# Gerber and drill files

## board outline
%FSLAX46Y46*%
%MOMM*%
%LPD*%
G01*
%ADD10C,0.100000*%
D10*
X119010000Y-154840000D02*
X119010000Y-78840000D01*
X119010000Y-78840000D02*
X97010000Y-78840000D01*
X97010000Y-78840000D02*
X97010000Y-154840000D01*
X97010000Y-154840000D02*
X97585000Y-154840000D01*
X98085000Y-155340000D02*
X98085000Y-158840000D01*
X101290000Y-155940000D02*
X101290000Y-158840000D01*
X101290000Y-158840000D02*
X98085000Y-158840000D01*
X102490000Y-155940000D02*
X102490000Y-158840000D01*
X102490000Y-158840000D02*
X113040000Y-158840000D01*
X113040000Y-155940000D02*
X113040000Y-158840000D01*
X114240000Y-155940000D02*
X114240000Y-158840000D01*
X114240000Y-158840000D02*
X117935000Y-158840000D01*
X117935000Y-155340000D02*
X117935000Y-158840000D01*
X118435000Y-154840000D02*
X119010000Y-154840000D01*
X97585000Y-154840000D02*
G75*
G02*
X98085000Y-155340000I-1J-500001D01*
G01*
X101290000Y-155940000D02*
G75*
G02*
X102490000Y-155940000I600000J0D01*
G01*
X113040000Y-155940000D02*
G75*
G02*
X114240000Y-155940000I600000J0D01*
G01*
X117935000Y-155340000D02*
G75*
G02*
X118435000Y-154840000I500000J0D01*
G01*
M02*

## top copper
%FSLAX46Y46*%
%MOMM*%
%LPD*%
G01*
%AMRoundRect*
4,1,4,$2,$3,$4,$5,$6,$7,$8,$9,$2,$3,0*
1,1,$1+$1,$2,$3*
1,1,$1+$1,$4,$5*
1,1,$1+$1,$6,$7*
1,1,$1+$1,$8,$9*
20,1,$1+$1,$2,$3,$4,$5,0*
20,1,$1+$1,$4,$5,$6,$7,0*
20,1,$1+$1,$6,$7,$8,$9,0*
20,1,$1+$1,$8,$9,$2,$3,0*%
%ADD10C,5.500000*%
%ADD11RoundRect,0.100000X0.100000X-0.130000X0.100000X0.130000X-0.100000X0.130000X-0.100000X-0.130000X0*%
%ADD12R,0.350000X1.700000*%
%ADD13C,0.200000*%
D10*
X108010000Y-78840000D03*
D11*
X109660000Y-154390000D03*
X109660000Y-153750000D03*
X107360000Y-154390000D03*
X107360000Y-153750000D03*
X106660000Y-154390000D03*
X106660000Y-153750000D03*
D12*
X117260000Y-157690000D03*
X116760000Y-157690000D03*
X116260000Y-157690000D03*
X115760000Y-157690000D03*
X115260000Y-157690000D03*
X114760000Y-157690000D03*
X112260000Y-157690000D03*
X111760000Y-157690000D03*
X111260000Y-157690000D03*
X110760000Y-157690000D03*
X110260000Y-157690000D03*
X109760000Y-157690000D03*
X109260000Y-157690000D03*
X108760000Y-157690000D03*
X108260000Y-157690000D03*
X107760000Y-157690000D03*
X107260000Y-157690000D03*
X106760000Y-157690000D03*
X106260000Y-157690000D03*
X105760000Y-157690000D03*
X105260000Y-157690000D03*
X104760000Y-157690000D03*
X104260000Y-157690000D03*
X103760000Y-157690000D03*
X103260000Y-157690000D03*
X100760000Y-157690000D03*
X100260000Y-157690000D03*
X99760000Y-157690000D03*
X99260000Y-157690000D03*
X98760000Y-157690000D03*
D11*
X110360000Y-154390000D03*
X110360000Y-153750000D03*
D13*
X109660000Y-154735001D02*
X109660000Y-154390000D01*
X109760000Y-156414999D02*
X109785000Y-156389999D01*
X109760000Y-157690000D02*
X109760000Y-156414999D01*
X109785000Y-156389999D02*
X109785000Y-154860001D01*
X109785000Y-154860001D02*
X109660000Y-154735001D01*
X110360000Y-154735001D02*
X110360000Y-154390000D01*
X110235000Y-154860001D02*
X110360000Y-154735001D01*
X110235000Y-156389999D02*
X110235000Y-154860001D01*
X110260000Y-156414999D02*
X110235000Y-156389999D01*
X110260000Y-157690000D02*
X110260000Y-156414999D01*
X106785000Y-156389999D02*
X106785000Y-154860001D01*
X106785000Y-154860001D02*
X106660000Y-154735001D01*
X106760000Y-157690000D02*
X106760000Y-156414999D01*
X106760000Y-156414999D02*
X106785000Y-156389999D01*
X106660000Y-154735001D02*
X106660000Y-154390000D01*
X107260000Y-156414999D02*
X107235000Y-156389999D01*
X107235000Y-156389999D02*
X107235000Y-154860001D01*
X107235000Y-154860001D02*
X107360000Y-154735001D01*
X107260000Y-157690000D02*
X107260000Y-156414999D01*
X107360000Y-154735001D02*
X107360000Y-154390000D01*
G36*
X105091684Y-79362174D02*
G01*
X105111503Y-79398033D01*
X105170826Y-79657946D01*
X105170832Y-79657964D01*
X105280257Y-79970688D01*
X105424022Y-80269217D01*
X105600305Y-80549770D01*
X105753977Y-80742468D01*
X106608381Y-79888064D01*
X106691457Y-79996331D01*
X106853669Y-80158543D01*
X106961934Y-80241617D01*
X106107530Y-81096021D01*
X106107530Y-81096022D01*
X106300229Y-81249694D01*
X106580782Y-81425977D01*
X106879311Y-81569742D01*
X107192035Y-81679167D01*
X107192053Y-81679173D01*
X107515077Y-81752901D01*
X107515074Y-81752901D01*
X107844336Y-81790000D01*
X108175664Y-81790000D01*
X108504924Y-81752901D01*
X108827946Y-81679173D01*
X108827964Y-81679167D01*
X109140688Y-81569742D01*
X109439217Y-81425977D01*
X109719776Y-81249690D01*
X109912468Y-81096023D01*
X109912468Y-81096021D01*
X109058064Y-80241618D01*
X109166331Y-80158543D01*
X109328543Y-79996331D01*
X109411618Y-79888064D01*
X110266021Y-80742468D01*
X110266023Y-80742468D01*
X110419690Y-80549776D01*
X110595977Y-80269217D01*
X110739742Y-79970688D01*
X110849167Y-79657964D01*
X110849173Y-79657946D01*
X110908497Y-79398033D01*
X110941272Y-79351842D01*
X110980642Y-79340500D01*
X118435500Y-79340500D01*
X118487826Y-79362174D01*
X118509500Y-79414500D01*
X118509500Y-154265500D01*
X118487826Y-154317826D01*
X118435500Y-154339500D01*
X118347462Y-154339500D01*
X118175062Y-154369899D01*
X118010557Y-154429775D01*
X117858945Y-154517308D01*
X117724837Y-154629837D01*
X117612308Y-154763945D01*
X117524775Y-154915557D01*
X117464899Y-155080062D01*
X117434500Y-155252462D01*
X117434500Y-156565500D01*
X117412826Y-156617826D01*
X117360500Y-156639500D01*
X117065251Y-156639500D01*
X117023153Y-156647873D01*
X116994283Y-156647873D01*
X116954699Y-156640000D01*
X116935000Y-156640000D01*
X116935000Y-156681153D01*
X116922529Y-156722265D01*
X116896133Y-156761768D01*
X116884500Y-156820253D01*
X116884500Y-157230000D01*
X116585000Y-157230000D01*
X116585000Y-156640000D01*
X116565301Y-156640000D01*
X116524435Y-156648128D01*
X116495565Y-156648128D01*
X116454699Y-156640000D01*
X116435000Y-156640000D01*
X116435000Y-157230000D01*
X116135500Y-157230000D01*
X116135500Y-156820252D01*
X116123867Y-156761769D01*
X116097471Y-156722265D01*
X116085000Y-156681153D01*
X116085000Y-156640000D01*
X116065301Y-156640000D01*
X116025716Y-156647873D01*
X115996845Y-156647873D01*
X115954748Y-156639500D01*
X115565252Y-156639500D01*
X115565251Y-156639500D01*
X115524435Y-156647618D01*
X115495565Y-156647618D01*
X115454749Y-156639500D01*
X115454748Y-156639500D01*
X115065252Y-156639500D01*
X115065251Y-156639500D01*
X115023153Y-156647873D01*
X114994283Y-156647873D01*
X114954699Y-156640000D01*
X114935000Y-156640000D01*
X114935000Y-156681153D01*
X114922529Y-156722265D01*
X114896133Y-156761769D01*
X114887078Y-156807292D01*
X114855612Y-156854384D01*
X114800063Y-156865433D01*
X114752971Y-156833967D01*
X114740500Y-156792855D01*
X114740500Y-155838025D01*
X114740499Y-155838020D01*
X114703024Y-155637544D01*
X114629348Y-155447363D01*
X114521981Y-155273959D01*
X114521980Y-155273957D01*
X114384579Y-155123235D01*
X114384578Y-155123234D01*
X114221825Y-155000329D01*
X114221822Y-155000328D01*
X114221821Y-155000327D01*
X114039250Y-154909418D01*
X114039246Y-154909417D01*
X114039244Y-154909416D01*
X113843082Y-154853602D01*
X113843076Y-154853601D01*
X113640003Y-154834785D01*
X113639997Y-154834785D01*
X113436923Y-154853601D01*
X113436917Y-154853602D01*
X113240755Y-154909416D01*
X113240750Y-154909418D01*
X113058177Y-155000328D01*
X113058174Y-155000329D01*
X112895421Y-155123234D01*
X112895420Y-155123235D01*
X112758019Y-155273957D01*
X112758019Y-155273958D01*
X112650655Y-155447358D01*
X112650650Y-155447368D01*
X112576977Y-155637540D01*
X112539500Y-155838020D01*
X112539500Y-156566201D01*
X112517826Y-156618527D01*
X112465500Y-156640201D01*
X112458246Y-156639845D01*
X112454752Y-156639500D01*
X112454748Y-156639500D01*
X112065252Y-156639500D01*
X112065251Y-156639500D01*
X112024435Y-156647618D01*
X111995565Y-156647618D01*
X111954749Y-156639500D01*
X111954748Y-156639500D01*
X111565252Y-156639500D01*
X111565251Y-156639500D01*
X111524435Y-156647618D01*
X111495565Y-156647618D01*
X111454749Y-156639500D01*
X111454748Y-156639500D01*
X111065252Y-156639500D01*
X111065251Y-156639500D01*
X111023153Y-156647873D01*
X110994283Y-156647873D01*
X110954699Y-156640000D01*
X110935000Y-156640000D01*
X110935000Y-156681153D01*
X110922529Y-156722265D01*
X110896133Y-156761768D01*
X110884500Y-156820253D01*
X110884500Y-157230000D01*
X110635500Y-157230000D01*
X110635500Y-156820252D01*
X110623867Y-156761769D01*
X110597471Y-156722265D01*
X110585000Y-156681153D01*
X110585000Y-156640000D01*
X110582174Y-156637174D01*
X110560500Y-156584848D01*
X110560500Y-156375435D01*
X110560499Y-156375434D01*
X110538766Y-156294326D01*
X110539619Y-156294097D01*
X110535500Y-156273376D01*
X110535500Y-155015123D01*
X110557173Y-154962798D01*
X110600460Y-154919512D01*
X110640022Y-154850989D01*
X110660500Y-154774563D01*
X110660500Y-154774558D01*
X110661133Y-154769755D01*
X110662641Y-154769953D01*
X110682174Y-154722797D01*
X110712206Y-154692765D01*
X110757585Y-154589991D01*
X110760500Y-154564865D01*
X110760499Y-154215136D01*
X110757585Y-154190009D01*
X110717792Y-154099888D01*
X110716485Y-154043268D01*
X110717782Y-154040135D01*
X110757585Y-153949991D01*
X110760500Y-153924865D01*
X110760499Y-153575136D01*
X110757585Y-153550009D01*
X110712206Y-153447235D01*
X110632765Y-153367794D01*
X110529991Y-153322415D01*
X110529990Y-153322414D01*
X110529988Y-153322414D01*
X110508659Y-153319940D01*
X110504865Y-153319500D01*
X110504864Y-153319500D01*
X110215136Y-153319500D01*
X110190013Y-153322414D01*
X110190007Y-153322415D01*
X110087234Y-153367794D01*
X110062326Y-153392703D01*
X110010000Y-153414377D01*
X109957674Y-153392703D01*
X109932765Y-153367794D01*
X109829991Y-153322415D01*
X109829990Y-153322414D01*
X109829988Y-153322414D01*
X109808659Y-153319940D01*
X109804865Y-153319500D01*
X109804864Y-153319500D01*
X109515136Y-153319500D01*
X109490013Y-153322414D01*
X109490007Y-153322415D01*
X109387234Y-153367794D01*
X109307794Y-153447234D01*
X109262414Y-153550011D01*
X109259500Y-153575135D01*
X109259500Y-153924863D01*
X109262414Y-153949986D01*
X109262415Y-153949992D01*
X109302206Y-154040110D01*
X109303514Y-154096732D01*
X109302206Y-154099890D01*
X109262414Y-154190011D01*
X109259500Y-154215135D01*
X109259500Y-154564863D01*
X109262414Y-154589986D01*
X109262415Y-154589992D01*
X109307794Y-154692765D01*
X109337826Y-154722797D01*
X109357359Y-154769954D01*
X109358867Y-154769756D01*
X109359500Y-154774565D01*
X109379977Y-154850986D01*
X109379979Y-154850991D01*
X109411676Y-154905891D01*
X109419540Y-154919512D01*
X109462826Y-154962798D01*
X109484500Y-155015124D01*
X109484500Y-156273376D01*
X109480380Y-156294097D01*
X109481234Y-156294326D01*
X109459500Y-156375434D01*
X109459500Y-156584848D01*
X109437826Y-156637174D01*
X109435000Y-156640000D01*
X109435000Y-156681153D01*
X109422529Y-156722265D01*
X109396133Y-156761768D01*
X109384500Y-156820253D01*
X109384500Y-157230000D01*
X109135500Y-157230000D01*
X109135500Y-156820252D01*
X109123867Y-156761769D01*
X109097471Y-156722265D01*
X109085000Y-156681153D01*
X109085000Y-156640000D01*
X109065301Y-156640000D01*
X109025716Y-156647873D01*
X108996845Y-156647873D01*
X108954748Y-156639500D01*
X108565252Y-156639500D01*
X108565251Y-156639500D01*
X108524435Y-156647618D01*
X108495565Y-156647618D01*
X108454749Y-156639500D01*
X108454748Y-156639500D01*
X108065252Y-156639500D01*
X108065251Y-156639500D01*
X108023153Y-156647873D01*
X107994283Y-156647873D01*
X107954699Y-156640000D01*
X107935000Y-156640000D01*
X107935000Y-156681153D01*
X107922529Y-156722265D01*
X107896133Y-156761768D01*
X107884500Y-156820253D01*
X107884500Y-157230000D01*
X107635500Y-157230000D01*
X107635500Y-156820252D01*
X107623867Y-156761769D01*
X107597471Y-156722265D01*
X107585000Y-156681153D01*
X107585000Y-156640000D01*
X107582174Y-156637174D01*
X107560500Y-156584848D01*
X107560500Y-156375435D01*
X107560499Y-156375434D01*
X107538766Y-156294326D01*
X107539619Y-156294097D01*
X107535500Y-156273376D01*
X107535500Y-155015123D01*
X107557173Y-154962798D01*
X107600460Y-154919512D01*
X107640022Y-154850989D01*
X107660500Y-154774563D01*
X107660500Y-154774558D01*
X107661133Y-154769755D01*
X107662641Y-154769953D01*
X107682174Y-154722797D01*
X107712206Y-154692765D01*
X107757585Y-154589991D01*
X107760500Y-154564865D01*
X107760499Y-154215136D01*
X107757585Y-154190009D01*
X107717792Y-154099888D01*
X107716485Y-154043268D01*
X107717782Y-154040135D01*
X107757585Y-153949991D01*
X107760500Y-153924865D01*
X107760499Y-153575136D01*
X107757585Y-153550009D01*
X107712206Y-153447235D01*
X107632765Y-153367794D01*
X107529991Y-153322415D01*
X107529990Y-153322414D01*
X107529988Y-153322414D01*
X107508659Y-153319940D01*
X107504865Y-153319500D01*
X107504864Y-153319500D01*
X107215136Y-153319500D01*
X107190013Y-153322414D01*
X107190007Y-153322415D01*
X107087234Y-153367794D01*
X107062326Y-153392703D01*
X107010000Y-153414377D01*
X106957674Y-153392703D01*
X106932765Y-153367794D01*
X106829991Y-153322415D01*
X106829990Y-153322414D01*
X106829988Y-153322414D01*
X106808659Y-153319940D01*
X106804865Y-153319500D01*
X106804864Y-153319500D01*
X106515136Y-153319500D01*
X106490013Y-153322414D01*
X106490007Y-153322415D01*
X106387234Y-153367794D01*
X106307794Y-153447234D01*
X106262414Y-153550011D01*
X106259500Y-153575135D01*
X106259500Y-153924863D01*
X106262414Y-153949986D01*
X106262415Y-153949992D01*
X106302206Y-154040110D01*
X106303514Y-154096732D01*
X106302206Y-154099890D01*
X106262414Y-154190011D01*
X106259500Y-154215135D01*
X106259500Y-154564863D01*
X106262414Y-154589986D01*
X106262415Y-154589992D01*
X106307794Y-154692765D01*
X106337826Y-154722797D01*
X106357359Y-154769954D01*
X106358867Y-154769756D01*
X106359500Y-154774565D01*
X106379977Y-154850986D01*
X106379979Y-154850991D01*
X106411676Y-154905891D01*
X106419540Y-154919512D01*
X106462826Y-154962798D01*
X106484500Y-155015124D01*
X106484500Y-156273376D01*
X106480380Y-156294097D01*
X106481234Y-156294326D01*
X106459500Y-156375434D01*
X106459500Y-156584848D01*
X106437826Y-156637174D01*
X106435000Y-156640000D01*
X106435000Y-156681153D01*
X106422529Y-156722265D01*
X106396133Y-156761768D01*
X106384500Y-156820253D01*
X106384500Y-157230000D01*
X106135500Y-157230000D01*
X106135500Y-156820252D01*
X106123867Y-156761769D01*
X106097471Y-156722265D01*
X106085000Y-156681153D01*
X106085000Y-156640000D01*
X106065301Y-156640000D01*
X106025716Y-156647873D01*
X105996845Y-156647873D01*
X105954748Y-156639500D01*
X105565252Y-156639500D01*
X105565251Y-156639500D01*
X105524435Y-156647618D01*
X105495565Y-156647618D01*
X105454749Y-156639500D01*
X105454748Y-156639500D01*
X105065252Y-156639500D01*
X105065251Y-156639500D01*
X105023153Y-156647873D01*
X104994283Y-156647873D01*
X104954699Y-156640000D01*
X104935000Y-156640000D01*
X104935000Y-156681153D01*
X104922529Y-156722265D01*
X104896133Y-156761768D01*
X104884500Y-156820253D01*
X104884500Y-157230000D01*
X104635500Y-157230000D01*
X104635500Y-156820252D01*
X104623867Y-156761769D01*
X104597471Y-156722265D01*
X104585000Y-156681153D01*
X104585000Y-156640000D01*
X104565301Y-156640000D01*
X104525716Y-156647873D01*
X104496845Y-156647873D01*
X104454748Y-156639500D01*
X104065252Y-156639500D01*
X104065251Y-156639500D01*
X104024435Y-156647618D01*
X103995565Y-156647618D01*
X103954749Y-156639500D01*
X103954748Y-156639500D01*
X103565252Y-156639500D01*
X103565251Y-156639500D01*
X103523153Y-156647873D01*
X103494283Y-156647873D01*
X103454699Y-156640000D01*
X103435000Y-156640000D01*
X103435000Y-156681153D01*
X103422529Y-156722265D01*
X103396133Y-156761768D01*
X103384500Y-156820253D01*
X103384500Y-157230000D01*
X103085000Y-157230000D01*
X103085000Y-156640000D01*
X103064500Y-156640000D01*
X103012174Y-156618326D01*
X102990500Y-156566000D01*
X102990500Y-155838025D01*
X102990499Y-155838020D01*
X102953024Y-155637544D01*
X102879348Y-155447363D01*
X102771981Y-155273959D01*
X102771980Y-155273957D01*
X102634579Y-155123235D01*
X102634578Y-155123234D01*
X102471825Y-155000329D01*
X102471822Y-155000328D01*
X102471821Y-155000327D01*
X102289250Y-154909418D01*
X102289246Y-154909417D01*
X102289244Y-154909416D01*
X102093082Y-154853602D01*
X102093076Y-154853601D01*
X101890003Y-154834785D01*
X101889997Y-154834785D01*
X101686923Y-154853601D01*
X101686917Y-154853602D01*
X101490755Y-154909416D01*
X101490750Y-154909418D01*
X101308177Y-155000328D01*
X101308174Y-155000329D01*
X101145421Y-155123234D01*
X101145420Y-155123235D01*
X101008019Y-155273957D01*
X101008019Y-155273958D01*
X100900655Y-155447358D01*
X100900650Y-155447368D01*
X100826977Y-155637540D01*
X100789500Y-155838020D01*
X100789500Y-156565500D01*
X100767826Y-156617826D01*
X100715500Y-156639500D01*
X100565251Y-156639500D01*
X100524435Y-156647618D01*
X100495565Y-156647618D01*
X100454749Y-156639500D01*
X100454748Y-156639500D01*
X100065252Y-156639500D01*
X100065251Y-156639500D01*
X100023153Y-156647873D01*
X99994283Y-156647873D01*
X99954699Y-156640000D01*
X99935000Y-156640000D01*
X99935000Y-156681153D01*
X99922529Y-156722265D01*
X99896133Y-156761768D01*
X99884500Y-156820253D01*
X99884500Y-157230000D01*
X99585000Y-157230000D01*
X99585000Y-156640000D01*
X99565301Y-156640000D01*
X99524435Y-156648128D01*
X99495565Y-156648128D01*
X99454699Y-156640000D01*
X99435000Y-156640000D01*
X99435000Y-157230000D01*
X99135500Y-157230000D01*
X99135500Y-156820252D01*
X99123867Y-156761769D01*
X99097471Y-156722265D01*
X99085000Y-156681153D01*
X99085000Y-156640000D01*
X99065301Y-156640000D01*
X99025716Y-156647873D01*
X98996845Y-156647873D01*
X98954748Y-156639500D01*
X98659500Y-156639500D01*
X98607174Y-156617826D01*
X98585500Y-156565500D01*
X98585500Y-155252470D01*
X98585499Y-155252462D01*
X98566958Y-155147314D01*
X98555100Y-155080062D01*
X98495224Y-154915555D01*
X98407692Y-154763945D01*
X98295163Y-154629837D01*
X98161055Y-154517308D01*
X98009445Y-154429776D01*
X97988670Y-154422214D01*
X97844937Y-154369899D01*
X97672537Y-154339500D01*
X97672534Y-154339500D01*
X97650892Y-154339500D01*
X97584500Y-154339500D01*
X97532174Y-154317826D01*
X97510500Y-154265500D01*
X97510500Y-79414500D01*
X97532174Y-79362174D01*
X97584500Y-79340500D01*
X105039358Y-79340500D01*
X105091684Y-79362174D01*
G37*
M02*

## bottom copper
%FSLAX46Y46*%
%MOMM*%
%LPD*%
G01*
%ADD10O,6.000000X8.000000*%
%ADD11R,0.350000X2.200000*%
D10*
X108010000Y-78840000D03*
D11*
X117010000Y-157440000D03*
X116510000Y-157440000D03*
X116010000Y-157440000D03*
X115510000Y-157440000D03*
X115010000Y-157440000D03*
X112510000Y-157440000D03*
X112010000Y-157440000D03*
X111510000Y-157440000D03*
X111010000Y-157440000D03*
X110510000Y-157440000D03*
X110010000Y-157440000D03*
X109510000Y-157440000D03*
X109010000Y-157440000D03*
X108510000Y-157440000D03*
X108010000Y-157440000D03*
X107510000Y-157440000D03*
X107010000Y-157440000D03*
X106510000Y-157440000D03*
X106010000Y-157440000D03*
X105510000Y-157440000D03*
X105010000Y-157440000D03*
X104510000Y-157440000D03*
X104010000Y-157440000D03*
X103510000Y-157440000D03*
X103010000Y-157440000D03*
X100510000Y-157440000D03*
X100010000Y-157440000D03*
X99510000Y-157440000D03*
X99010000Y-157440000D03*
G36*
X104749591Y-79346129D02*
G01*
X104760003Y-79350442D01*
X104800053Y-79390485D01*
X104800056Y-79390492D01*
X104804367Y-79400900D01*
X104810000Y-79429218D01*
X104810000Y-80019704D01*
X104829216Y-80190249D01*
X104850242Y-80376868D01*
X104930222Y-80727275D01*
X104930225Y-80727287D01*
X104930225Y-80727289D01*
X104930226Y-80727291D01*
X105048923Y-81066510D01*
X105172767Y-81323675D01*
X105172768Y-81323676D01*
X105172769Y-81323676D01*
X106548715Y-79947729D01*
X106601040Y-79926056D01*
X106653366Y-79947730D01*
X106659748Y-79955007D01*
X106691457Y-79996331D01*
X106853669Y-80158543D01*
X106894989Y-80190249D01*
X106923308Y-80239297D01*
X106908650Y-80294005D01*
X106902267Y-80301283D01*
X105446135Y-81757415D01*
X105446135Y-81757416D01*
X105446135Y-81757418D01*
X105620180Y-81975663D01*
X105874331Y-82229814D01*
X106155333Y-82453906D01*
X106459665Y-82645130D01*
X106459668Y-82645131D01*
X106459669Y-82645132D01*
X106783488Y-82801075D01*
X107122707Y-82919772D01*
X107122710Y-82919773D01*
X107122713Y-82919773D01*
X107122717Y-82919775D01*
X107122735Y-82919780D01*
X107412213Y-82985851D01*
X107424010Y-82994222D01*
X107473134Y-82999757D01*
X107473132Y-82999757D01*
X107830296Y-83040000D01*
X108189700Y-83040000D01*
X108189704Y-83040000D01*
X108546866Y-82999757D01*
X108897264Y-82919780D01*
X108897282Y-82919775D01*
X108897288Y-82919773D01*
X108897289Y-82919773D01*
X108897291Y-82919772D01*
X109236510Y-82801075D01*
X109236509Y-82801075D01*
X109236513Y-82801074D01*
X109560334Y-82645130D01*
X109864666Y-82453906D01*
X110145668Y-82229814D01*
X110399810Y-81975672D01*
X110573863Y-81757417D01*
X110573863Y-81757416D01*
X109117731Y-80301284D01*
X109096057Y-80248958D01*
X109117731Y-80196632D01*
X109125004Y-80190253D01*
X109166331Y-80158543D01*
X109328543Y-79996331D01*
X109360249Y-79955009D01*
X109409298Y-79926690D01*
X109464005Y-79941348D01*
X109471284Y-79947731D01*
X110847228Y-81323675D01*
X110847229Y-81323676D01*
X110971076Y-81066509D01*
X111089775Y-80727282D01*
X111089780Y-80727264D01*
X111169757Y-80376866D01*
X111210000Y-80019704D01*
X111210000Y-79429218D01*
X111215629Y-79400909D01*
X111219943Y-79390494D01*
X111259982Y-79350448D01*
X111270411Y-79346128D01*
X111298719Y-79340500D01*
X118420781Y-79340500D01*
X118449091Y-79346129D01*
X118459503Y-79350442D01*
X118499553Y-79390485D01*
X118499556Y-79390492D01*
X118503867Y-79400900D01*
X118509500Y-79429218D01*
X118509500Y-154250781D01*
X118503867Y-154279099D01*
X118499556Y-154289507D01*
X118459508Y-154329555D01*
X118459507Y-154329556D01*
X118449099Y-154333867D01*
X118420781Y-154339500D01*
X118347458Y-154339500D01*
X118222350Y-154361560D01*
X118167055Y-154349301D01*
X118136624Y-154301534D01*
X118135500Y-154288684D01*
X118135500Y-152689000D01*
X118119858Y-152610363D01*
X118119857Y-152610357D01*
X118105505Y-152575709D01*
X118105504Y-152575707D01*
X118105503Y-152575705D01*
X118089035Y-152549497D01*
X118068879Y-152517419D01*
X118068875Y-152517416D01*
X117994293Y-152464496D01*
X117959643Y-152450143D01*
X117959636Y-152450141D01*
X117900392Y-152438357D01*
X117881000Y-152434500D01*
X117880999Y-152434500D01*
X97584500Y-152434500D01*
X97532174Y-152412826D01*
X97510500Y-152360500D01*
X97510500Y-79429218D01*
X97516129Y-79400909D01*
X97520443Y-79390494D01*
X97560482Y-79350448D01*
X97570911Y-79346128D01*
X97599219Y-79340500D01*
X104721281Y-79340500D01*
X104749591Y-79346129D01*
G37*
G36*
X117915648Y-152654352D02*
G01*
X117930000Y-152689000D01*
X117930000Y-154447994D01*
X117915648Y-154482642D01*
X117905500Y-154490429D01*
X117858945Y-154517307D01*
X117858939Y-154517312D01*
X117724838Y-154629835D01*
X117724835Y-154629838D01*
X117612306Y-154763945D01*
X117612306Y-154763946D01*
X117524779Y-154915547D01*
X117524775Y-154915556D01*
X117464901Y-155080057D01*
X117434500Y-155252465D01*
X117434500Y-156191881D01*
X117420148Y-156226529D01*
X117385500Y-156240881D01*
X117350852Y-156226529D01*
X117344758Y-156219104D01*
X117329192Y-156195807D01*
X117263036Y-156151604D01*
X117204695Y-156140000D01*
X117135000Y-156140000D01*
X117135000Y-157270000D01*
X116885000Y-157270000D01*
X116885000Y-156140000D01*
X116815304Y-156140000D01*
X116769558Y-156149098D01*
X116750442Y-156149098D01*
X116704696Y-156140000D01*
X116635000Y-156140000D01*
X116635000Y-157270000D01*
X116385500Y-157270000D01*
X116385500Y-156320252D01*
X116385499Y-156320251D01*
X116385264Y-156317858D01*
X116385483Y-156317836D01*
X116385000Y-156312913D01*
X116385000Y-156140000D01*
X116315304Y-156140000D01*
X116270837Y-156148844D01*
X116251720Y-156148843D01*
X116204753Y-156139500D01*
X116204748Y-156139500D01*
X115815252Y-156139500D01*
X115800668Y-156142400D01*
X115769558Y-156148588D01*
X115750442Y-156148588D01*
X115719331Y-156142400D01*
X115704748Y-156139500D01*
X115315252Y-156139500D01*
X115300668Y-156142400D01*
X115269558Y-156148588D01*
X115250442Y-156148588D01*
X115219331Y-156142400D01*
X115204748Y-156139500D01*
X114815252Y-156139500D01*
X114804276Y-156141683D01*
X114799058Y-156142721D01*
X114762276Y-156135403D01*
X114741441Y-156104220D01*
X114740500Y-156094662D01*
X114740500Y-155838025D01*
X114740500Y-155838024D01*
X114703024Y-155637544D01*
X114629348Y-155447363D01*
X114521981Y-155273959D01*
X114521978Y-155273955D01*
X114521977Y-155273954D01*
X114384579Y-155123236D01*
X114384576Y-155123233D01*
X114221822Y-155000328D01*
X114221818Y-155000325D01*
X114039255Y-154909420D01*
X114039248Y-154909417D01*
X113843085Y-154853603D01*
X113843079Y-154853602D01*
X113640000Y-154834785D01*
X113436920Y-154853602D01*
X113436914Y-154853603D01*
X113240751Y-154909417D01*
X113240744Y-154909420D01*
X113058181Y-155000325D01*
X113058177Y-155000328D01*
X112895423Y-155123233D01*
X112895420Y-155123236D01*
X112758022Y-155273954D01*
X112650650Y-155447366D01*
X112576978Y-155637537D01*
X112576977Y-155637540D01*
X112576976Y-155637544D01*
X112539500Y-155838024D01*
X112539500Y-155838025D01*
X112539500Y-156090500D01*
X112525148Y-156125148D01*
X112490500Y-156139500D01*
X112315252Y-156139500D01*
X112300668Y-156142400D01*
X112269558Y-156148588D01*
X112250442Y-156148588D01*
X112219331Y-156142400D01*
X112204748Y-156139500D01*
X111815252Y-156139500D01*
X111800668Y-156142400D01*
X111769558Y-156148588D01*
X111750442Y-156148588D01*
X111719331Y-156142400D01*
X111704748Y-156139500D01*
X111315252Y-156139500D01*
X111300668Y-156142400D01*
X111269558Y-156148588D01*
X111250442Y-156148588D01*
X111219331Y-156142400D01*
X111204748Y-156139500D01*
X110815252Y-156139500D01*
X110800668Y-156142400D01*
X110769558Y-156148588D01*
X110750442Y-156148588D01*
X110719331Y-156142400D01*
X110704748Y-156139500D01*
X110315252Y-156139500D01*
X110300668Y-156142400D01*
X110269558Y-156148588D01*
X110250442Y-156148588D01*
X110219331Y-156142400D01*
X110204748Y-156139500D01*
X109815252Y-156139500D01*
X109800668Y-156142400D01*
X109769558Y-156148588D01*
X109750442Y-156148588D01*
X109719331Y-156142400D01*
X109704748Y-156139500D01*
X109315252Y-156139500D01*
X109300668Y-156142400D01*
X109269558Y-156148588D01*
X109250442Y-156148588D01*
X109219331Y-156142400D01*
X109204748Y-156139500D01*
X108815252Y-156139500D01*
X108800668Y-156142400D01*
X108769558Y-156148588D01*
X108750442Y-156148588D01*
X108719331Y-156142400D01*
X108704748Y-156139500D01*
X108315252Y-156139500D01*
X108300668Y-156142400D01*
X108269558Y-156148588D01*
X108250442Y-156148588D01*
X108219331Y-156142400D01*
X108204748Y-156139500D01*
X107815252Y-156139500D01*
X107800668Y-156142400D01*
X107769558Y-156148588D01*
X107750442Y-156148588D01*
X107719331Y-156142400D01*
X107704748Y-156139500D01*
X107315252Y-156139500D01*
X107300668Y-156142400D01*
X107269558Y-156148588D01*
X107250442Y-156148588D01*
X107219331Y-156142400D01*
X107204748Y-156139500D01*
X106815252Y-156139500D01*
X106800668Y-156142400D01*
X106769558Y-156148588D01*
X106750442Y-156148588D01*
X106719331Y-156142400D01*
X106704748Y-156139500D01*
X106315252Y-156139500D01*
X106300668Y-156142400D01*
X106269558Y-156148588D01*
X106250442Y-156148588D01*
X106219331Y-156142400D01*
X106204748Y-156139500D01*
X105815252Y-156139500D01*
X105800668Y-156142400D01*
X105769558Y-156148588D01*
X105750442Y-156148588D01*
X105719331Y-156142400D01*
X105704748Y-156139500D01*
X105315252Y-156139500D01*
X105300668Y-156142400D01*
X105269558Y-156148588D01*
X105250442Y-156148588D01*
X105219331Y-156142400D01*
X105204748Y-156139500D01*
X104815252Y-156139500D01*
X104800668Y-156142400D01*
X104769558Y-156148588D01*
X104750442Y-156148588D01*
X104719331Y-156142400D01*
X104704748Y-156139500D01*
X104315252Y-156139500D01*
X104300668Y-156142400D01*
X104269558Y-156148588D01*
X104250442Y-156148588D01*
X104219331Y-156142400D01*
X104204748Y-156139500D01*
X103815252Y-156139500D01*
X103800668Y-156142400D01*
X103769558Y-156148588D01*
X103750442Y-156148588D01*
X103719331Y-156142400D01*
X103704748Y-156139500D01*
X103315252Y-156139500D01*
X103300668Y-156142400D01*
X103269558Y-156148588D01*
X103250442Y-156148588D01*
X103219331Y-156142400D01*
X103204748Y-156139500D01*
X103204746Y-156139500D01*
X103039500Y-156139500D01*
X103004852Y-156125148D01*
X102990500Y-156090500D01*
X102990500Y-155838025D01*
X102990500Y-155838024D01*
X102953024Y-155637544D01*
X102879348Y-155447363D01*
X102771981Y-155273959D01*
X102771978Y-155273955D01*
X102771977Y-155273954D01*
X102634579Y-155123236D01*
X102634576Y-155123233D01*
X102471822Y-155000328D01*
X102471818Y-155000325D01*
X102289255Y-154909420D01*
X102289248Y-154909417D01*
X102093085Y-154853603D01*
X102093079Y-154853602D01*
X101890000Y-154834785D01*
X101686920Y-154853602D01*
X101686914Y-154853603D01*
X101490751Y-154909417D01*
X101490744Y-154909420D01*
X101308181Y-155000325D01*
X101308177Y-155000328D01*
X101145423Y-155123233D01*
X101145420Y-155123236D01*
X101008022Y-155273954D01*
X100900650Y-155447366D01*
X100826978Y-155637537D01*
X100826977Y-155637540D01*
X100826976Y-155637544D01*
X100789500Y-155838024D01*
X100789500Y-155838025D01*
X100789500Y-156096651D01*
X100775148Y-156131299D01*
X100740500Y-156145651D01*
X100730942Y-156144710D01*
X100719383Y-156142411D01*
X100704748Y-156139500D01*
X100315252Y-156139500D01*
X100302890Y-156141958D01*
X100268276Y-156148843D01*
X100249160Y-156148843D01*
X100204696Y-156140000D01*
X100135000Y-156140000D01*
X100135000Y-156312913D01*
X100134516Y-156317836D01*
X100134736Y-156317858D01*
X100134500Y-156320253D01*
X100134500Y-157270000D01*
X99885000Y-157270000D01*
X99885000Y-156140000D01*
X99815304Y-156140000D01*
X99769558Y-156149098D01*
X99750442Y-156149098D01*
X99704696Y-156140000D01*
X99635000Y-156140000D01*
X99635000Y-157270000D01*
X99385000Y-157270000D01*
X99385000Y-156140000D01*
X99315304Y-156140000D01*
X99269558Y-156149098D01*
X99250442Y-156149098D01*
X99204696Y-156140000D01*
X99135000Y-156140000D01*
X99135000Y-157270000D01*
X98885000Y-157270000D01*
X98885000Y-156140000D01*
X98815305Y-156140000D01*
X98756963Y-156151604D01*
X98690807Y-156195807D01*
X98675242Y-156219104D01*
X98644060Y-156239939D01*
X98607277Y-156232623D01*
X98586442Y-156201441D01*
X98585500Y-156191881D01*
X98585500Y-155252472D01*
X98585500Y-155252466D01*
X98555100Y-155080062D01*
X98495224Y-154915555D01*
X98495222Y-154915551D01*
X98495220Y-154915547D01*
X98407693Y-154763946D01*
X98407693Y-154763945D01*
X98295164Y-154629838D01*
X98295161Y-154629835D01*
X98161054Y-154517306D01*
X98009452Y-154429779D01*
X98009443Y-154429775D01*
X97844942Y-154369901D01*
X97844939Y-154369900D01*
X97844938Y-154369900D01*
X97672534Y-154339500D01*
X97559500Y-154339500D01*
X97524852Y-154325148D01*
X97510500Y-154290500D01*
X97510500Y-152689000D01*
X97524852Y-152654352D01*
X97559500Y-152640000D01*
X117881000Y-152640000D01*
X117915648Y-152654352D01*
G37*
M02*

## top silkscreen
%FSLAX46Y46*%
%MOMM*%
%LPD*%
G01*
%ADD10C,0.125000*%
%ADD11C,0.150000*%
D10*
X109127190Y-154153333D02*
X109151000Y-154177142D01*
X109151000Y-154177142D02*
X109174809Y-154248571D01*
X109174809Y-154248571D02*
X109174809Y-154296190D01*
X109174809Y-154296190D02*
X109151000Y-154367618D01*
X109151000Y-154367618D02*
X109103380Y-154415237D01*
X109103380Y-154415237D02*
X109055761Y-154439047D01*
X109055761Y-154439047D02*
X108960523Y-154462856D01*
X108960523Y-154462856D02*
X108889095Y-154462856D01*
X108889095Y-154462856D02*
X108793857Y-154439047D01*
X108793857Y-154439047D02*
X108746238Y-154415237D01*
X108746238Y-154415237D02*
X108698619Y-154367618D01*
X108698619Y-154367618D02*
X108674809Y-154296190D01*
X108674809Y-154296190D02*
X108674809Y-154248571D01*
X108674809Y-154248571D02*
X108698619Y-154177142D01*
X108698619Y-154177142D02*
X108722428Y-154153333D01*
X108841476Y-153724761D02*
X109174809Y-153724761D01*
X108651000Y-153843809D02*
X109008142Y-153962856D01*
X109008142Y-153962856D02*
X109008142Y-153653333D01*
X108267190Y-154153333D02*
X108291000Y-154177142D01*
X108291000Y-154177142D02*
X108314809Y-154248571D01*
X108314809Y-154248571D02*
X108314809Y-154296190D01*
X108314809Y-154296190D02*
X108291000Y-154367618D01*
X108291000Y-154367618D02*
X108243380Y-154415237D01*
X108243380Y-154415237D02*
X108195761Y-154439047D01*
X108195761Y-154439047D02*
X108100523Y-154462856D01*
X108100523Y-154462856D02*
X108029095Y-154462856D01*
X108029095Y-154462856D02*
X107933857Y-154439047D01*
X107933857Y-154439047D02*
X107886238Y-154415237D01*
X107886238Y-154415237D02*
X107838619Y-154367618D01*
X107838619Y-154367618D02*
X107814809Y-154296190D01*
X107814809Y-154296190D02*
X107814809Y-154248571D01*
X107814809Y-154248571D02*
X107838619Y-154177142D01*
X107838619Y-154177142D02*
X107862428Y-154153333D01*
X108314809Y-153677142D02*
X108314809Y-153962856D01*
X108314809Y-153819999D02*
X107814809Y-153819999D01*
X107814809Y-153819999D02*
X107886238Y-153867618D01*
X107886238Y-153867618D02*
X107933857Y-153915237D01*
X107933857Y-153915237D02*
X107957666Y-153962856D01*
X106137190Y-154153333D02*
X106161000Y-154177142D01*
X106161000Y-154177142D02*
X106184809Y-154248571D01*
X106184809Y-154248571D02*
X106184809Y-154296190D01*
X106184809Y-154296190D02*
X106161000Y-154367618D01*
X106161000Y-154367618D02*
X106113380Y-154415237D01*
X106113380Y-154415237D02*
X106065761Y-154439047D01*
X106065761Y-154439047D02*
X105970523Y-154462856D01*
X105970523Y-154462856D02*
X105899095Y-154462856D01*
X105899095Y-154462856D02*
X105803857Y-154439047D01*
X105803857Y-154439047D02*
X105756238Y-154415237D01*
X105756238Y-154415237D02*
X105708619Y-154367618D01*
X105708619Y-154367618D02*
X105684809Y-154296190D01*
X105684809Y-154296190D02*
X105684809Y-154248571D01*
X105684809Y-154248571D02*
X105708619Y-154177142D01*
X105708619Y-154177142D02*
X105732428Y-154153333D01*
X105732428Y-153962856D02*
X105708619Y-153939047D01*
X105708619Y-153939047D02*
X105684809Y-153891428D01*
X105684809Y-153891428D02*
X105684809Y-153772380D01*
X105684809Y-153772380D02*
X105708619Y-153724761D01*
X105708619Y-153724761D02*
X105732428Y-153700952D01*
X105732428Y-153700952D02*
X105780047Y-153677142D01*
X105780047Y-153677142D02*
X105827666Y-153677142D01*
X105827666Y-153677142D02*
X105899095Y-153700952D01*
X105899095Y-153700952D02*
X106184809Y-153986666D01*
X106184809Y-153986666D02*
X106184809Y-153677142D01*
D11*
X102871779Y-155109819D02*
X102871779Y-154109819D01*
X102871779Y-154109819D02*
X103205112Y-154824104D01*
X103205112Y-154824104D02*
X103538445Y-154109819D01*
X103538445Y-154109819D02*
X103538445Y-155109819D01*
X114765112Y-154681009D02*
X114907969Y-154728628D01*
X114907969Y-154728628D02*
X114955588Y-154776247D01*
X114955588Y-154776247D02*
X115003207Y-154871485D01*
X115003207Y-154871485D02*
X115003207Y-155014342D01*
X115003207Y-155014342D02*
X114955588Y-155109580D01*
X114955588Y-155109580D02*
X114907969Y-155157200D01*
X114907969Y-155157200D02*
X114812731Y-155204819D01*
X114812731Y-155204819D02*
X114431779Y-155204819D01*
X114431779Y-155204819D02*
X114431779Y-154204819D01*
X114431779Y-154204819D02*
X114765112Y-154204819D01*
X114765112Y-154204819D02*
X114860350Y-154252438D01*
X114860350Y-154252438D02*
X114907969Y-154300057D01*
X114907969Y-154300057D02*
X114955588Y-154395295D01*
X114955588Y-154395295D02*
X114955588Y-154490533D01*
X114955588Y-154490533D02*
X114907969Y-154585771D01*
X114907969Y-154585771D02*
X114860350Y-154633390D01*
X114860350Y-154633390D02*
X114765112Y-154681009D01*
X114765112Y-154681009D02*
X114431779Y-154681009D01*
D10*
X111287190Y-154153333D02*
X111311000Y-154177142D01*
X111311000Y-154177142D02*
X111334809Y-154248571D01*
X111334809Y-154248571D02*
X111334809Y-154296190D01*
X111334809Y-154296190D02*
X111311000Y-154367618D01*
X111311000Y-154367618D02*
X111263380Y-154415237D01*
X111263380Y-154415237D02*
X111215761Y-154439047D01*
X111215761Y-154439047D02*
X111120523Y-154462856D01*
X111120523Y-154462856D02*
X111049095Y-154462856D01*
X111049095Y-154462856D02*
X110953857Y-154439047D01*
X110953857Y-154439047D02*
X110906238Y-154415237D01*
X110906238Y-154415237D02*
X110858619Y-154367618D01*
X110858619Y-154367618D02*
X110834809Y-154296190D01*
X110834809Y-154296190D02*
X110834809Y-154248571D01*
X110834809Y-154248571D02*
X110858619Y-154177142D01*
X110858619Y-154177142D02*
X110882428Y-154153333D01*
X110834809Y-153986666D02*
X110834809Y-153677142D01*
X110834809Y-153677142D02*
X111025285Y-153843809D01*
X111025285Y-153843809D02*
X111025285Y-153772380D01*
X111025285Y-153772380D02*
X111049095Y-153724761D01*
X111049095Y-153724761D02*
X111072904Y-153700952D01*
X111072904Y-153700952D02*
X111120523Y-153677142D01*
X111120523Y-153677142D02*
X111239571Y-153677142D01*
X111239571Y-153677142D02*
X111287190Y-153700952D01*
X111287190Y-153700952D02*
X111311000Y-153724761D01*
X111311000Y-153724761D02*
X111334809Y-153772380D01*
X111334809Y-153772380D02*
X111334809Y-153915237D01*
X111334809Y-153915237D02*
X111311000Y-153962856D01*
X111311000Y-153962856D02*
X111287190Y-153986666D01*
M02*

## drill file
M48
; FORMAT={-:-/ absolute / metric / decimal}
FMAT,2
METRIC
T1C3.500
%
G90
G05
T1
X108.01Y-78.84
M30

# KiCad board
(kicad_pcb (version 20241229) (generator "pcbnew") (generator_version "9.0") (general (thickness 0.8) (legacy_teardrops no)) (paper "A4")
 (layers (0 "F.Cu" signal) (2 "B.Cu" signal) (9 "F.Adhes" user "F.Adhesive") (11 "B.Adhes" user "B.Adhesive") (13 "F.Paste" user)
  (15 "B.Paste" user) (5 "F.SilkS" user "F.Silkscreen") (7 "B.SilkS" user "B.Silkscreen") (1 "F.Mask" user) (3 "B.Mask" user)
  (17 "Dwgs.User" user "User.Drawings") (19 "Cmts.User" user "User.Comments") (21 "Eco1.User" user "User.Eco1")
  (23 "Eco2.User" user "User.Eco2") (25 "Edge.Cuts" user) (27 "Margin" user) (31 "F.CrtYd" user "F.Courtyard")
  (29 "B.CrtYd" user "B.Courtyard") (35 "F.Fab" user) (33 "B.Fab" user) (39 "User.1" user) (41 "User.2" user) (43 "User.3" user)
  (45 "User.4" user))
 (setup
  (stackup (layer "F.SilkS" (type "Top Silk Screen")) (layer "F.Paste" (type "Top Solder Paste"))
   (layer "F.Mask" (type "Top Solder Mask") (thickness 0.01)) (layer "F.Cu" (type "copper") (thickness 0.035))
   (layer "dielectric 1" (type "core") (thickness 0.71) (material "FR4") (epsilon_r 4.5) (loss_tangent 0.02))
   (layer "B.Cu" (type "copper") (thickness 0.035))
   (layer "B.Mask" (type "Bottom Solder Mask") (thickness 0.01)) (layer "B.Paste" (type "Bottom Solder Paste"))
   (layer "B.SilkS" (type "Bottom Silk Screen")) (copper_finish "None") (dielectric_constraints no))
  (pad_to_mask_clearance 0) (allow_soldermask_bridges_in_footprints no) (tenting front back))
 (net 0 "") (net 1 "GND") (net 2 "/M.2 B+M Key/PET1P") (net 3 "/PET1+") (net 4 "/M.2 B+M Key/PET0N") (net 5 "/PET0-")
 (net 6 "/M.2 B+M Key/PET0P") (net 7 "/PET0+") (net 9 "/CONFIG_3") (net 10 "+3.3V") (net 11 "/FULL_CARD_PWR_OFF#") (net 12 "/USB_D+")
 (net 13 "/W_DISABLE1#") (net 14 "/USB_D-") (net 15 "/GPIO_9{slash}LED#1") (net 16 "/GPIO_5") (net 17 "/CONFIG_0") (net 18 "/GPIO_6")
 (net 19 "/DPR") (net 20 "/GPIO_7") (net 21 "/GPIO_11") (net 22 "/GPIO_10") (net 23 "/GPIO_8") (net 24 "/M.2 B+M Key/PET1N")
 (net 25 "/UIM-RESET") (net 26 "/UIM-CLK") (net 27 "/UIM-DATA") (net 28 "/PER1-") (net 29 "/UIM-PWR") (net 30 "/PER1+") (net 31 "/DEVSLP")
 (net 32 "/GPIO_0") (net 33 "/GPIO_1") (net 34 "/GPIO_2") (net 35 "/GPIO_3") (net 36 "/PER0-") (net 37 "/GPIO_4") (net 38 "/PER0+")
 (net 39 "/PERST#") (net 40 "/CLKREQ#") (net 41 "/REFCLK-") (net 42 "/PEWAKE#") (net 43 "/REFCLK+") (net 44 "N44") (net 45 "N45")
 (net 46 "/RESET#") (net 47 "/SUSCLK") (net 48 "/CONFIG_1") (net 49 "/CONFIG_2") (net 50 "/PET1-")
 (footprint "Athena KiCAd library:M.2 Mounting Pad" (layer "F.Cu") (at 108.01 78.84)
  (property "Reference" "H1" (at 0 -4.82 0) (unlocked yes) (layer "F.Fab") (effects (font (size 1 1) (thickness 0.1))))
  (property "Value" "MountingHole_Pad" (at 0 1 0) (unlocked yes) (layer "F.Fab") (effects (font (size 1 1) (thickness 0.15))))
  (pad "1" thru_hole circle (at 0 0) (size 5.5 5.5) (drill 3.5) (layers "*.Cu" "*.Mask") (remove_unused_layers no) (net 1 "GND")
   (padstack (mode front_inner_back)
    (layer "Inner" (shape circle) (size 5.5 5.5) (zone_connect -1))
    (layer "B.Cu" (shape oval) (size 6 8) (thermal_bridge_angle 45) (zone_connect -1)))))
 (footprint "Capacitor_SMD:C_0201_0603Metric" (layer "F.Cu") (at 109.66 154.07 90)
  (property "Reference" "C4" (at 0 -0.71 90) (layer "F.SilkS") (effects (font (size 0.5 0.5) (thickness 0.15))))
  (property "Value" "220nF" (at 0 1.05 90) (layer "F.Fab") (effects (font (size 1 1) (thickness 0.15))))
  (pad "" smd roundrect (at -0.345 0 90) (size 0.318 0.36) (layers "F.Paste") (roundrect_rratio 0.25))
  (pad "" smd roundrect (at 0.345 0 90) (size 0.318 0.36) (layers "F.Paste") (roundrect_rratio 0.25))
  (pad "1" smd roundrect (at -0.32 0 90) (size 0.46 0.4) (layers "F.Cu" "F.Mask") (roundrect_rratio 0.25) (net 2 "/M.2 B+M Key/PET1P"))
  (pad "2" smd roundrect (at 0.32 0 90) (size 0.46 0.4) (layers "F.Cu" "F.Mask") (roundrect_rratio 0.25) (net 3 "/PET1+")))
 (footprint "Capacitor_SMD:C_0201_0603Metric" (layer "F.Cu") (at 107.36 154.07 90)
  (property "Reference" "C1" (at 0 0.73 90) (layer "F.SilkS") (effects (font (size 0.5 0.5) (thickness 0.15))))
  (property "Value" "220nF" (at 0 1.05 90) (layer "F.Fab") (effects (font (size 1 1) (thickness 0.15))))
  (pad "" smd roundrect (at -0.345 0 90) (size 0.318 0.36) (layers "F.Paste") (roundrect_rratio 0.25))
  (pad "" smd roundrect (at 0.345 0 90) (size 0.318 0.36) (layers "F.Paste") (roundrect_rratio 0.25))
  (pad "1" smd roundrect (at -0.32 0 90) (size 0.46 0.4) (layers "F.Cu" "F.Mask") (roundrect_rratio 0.25) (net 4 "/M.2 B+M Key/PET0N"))
  (pad "2" smd roundrect (at 0.32 0 90) (size 0.46 0.4) (layers "F.Cu" "F.Mask") (roundrect_rratio 0.25) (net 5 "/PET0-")))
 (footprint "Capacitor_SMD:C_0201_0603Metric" (layer "F.Cu") (at 106.66 154.07 90)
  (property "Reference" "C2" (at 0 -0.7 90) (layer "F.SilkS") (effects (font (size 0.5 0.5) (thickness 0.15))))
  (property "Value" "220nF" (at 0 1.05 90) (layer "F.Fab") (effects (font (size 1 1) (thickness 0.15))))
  (pad "" smd roundrect (at -0.345 0 90) (size 0.318 0.36) (layers "F.Paste") (roundrect_rratio 0.25))
  (pad "" smd roundrect (at 0.345 0 90) (size 0.318 0.36) (layers "F.Paste") (roundrect_rratio 0.25))
  (pad "1" smd roundrect (at -0.32 0 90) (size 0.46 0.4) (layers "F.Cu" "F.Mask") (roundrect_rratio 0.25) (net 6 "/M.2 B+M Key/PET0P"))
  (pad "2" smd roundrect (at 0.32 0 90) (size 0.46 0.4) (layers "F.Cu" "F.Mask") (roundrect_rratio 0.25) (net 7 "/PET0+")))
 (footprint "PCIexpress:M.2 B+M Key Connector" (layer "F.Cu") (at 108.01 157.73)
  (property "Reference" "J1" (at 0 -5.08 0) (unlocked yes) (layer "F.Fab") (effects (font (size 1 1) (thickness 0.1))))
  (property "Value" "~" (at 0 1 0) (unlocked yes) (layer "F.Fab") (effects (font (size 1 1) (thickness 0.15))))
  (fp_line (start -11 -2.89) (end -10.425 -2.89) (stroke (width 0.1) (type default)) (layer "Edge.Cuts") (net 8))
  (fp_line (start -9.925 -2.39) (end -9.925 1.11) (stroke (width 0.1) (type default)) (layer "Edge.Cuts") (net 8))
  (fp_line (start -6.72 -1.79) (end -6.72 1.11) (stroke (width 0.1) (type default)) (layer "Edge.Cuts") (net 8))
  (fp_line (start -6.72 1.11) (end -9.925 1.11) (stroke (width 0.1) (type default)) (layer "Edge.Cuts") (net 8))
  (fp_line (start -5.52 -1.79) (end -5.52 1.11) (stroke (width 0.1) (type default)) (layer "Edge.Cuts") (net 8))
  (fp_line (start -5.52 1.11) (end 5.03 1.11) (stroke (width 0.1) (type default)) (layer "Edge.Cuts") (net 8))
  (fp_line (start 5.03 -1.79) (end 5.03 1.11) (stroke (width 0.1) (type default)) (layer "Edge.Cuts") (net 8))
  (fp_line (start 6.23 -1.79) (end 6.23 1.11) (stroke (width 0.1) (type default)) (layer "Edge.Cuts") (net 8))
  (fp_line (start 6.23 1.11) (end 9.925 1.11) (stroke (width 0.1) (type default)) (layer "Edge.Cuts") (net 8))
  (fp_line (start 9.925 -2.39) (end 9.925 1.11) (stroke (width 0.1) (type default)) (layer "Edge.Cuts") (net 8))
  (fp_line (start 10.425 -2.89) (end 11 -2.89) (stroke (width 0.1) (type default)) (layer "Edge.Cuts") (net 8))
  (fp_arc (start -10.425 -2.89) (mid -10.071447 -2.743553) (end -9.925 -2.39) (stroke (width 0.1) (type default)) (layer "Edge.Cuts")
   (net 8))
  (fp_arc (start -6.72 -1.79) (mid -6.12 -2.39) (end -5.52 -1.79) (stroke (width 0.1) (type default)) (layer "Edge.Cuts") (net 8))
  (fp_arc (start 5.03 -1.79) (mid 5.63 -2.39) (end 6.23 -1.79) (stroke (width 0.1) (type default)) (layer "Edge.Cuts") (net 8))
  (fp_arc (start 9.925 -2.39) (mid 10.071447 -2.743553) (end 10.425 -2.89) (stroke (width 0.1) (type default)) (layer "Edge.Cuts") (net 8))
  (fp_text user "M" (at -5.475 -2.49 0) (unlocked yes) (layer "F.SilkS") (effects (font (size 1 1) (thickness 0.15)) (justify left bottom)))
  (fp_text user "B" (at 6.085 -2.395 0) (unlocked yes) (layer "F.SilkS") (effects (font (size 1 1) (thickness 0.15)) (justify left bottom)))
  (pad "1" smd rect (at 9.25 -0.04 180) (size 0.35 1.7) (layers "F.Cu") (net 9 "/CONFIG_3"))
  (pad "2" smd rect (at 9 -0.29 180) (size 0.35 2.2) (layers "B.Cu") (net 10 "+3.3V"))
  (pad "3" smd rect (at 8.75 -0.04 180) (size 0.35 1.7) (layers "F.Cu") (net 1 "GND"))
  (pad "4" smd rect (at 8.5 -0.29 180) (size 0.35 2.2) (layers "B.Cu") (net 10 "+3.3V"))
  (pad "5" smd rect (at 8.25 -0.04 180) (size 0.35 1.7) (layers "F.Cu") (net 1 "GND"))
  (pad "6" smd rect (at 8 -0.29 180) (size 0.35 2.2) (layers "B.Cu") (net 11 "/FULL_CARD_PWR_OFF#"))
  (pad "7" smd rect (at 7.75 -0.04 180) (size 0.35 1.7) (layers "F.Cu") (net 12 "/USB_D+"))
  (pad "8" smd rect (at 7.5 -0.29 180) (size 0.35 2.2) (layers "B.Cu") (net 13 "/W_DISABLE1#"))
  (pad "9" smd rect (at 7.25 -0.04 180) (size 0.35 1.7) (layers "F.Cu") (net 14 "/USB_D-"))
  (pad "10" smd rect (at 7 -0.29 180) (size 0.35 2.2) (layers "B.Cu") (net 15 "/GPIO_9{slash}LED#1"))
  (pad "11" smd rect (at 6.75 -0.04 180) (size 0.35 1.7) (layers "F.Cu") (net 1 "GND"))
  (pad "20" smd rect (at 4.5 -0.29 180) (size 0.35 2.2) (layers "B.Cu") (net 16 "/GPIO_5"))
  (pad "21" smd rect (at 4.25 -0.04 180) (size 0.35 1.7) (layers "F.Cu") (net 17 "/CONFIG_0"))
  (pad "22" smd rect (at 4 -0.29 180) (size 0.35 2.2) (layers "B.Cu") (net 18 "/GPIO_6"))
  (pad "23" smd rect (at 3.75 -0.04 180) (size 0.35 1.7) (layers "F.Cu") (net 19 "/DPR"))
  (pad "24" smd rect (at 3.5 -0.29 180) (size 0.35 2.2) (layers "B.Cu") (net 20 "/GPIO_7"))
  (pad "25" smd rect (at 3.25 -0.04 180) (size 0.35 1.7) (layers "F.Cu") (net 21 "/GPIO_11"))
  (pad "26" smd rect (at 3 -0.29 180) (size 0.35 2.2) (layers "B.Cu") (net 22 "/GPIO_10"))
  (pad "27" smd rect (at 2.75 -0.04 180) (size 0.35 1.7) (layers "F.Cu") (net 1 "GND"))
  (pad "28" smd rect (at 2.5 -0.29 180) (size 0.35 2.2) (layers "B.Cu") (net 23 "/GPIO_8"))
  (pad "29" smd rect (at 2.25 -0.04 180) (size 0.35 1.7) (layers "F.Cu") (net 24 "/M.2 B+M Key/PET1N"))
  (pad "30" smd rect (at 2 -0.29 180) (size 0.35 2.2) (layers "B.Cu") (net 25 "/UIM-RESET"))
  (pad "31" smd rect (at 1.75 -0.04 180) (size 0.35 1.7) (layers "F.Cu") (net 2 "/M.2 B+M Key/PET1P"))
  (pad "32" smd rect (at 1.5 -0.29 180) (size 0.35 2.2) (layers "B.Cu") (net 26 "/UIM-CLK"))
  (pad "33" smd rect (at 1.25 -0.04 180) (size 0.35 1.7) (layers "F.Cu") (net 1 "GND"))
  (pad "34" smd rect (at 1 -0.29 180) (size 0.35 2.2) (layers "B.Cu") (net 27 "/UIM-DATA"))
  (pad "35" smd rect (at 0.75 -0.04 180) (size 0.35 1.7) (layers "F.Cu") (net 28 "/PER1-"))
  (pad "36" smd rect (at 0.5 -0.29 180) (size 0.35 2.2) (layers "B.Cu") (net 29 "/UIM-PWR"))
  (pad "37" smd rect (at 0.25 -0.04 180) (size 0.35 1.7) (layers "F.Cu") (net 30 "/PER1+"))
  (pad "38" smd rect (at 0 -0.29 180) (size 0.35 2.2) (layers "B.Cu") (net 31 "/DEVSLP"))
  (pad "39" smd rect (at -0.25 -0.04 180) (size 0.35 1.7) (layers "F.Cu") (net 1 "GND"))
  (pad "40" smd rect (at -0.5 -0.29 180) (size 0.35 2.2) (layers "B.Cu") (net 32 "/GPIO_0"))
  (pad "41" smd rect (at -0.75 -0.04 180) (size 0.35 1.7) (layers "F.Cu") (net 4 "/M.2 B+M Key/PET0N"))
  (pad "42" smd rect (at -1 -0.29 180) (size 0.35 2.2) (layers "B.Cu") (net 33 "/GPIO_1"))
  (pad "43" smd rect (at -1.25 -0.04 180) (size 0.35 1.7) (layers "F.Cu") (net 6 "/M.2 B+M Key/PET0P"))
  (pad "44" smd rect (at -1.5 -0.29 180) (size 0.35 2.2) (layers "B.Cu") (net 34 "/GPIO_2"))
  (pad "45" smd rect (at -1.75 -0.04 180) (size 0.35 1.7) (layers "F.Cu") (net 1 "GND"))
  (pad "46" smd rect (at -2 -0.29 180) (size 0.35 2.2) (layers "B.Cu") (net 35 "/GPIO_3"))
  (pad "47" smd rect (at -2.25 -0.04 180) (size 0.35 1.7) (layers "F.Cu") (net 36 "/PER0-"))
  (pad "48" smd rect (at -2.5 -0.29 180) (size 0.35 2.2) (layers "B.Cu") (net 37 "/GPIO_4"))
  (pad "49" smd rect (at -2.75 -0.04 180) (size 0.35 1.7) (layers "F.Cu") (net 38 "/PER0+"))
  (pad "50" smd rect (at -3 -0.29 180) (size 0.35 2.2) (layers "B.Cu") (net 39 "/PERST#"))
  (pad "51" smd rect (at -3.25 -0.04 180) (size 0.35 1.7) (layers "F.Cu") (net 1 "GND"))
  (pad "52" smd rect (at -3.5 -0.29 180) (size 0.35 2.2) (layers "B.Cu") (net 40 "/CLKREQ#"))
  (pad "53" smd rect (at -3.75 -0.04 180) (size 0.35 1.7) (layers "F.Cu") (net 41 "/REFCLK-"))
  (pad "54" smd rect (at -4 -0.29 180) (size 0.35 2.2) (layers "B.Cu") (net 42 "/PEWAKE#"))
  (pad "55" smd rect (at -4.25 -0.04 180) (size 0.35 1.7) (layers "F.Cu") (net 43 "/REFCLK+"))
  (pad "56" smd rect (at -4.5 -0.29 180) (size 0.35 2.2) (layers "B.Cu") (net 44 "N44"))
  (pad "57" smd rect (at -4.75 -0.04 180) (size 0.35 1.7) (layers "F.Cu") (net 1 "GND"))
  (pad "58" smd rect (at -5 -0.29 180) (size 0.35 2.2) (layers "B.Cu") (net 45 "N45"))
  (pad "67" smd rect (at -7.25 -0.04 180) (size 0.35 1.7) (layers "F.Cu") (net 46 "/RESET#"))
  (pad "68" smd rect (at -7.5 -0.29 180) (size 0.35 2.2) (layers "B.Cu") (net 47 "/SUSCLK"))
  (pad "69" smd rect (at -7.75 -0.04 180) (size 0.35 1.7) (layers "F.Cu") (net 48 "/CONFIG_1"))
  (pad "70" smd rect (at -8 -0.29 180) (size 0.35 2.2) (layers "B.Cu") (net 10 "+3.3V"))
  (pad "71" smd rect (at -8.25 -0.04 180) (size 0.35 1.7) (layers "F.Cu") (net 1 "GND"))
  (pad "72" smd rect (at -8.5 -0.29 180) (size 0.35 2.2) (layers "B.Cu") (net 10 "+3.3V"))
  (pad "73" smd rect (at -8.75 -0.04 180) (size 0.35 1.7) (layers "F.Cu") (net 1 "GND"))
  (pad "74" smd rect (at -9 -0.29 180) (size 0.35 2.2) (layers "B.Cu") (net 10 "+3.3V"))
  (pad "75" smd rect (at -9.25 -0.04 180) (size 0.35 1.7) (layers "F.Cu") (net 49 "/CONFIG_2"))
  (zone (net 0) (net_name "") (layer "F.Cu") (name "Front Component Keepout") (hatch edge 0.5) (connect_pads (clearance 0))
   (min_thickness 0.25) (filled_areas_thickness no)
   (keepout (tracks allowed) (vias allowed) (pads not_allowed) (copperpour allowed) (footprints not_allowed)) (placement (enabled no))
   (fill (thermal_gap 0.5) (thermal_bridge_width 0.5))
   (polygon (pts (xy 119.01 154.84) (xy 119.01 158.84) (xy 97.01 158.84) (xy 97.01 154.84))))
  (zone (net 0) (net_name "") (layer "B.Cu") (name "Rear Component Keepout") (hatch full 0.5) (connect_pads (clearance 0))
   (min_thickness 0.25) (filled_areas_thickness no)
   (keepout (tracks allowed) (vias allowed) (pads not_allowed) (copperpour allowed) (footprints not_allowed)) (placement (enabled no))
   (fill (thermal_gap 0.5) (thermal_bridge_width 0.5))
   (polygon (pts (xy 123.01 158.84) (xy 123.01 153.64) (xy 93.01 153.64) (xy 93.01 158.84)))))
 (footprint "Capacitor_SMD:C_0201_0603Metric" (layer "F.Cu") (at 110.36 154.07 90)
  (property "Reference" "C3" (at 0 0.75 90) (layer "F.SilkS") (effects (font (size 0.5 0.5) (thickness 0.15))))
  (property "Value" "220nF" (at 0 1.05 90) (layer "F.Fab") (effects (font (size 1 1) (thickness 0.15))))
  (pad "" smd roundrect (at -0.345 0 90) (size 0.318 0.36) (layers "F.Paste") (roundrect_rratio 0.25))
  (pad "" smd roundrect (at 0.345 0 90) (size 0.318 0.36) (layers "F.Paste") (roundrect_rratio 0.25))
  (pad "1" smd roundrect (at -0.32 0 90) (size 0.46 0.4) (layers "F.Cu" "F.Mask") (roundrect_rratio 0.25) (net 24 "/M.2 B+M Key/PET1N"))
  (pad "2" smd roundrect (at 0.32 0 90) (size 0.46 0.4) (layers "F.Cu" "F.Mask") (roundrect_rratio 0.25) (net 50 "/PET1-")))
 (gr_line (start 119.01 154.84) (end 119.01 78.84) (stroke (width 0.1) (type default)) (layer "Edge.Cuts"))
 (gr_line (start 119.01 78.84) (end 97.01 78.84) (stroke (width 0.1) (type default)) (layer "Edge.Cuts"))
 (gr_line (start 97.01 78.84) (end 97.01 154.84) (stroke (width 0.1) (type default)) (layer "Edge.Cuts"))
 (segment (start 109.66 154.735001) (end 109.66 154.39) (width 0.2) (layer "F.Cu") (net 2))
 (segment (start 109.76 156.414999) (end 109.785 156.389999) (width 0.2) (layer "F.Cu") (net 2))
 (segment (start 109.76 157.69) (end 109.76 156.414999) (width 0.2) (layer "F.Cu") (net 2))
 (segment (start 109.785 156.389999) (end 109.785 154.860001) (width 0.2) (layer "F.Cu") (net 2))
 (segment (start 109.785 154.860001) (end 109.66 154.735001) (width 0.2) (layer "F.Cu") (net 2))
 (segment (start 110.36 154.735001) (end 110.36 154.39) (width 0.2) (layer "F.Cu") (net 24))
 (segment (start 110.235 154.860001) (end 110.36 154.735001) (width 0.2) (layer "F.Cu") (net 24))
 (segment (start 110.235 156.389999) (end 110.235 154.860001) (width 0.2) (layer "F.Cu") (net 24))
 (segment (start 110.26 156.414999) (end 110.235 156.389999) (width 0.2) (layer "F.Cu") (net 24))
 (segment (start 110.26 157.69) (end 110.26 156.414999) (width 0.2) (layer "F.Cu") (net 24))
 (segment (start 106.785 156.389999) (end 106.785 154.860001) (width 0.2) (layer "F.Cu") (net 6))
 (segment (start 106.785 154.860001) (end 106.66 154.735001) (width 0.2) (layer "F.Cu") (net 6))
 (segment (start 106.76 157.69) (end 106.76 156.414999) (width 0.2) (layer "F.Cu") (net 6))
 (segment (start 106.76 156.414999) (end 106.785 156.389999) (width 0.2) (layer "F.Cu") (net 6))
 (segment (start 106.66 154.735001) (end 106.66 154.39) (width 0.2) (layer "F.Cu") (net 6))
 (segment (start 107.26 156.414999) (end 107.235 156.389999) (width 0.2) (layer "F.Cu") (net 4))
 (segment (start 107.235 156.389999) (end 107.235 154.860001) (width 0.2) (layer "F.Cu") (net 4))
 (segment (start 107.235 154.860001) (end 107.36 154.735001) (width 0.2) (layer "F.Cu") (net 4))
 (segment (start 107.26 157.69) (end 107.26 156.414999) (width 0.2) (layer "F.Cu") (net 4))
 (segment (start 107.36 154.735001) (end 107.36 154.39) (width 0.2) (layer "F.Cu") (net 4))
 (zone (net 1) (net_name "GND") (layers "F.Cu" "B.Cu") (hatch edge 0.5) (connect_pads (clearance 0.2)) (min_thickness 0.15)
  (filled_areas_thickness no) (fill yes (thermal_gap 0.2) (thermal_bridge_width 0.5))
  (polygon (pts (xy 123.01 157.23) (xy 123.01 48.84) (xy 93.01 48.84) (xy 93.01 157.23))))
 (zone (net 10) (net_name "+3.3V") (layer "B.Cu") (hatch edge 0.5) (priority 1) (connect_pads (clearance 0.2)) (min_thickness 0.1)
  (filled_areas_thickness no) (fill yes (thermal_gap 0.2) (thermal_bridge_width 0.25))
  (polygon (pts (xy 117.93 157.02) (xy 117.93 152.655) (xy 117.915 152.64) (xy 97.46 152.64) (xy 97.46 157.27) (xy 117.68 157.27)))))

